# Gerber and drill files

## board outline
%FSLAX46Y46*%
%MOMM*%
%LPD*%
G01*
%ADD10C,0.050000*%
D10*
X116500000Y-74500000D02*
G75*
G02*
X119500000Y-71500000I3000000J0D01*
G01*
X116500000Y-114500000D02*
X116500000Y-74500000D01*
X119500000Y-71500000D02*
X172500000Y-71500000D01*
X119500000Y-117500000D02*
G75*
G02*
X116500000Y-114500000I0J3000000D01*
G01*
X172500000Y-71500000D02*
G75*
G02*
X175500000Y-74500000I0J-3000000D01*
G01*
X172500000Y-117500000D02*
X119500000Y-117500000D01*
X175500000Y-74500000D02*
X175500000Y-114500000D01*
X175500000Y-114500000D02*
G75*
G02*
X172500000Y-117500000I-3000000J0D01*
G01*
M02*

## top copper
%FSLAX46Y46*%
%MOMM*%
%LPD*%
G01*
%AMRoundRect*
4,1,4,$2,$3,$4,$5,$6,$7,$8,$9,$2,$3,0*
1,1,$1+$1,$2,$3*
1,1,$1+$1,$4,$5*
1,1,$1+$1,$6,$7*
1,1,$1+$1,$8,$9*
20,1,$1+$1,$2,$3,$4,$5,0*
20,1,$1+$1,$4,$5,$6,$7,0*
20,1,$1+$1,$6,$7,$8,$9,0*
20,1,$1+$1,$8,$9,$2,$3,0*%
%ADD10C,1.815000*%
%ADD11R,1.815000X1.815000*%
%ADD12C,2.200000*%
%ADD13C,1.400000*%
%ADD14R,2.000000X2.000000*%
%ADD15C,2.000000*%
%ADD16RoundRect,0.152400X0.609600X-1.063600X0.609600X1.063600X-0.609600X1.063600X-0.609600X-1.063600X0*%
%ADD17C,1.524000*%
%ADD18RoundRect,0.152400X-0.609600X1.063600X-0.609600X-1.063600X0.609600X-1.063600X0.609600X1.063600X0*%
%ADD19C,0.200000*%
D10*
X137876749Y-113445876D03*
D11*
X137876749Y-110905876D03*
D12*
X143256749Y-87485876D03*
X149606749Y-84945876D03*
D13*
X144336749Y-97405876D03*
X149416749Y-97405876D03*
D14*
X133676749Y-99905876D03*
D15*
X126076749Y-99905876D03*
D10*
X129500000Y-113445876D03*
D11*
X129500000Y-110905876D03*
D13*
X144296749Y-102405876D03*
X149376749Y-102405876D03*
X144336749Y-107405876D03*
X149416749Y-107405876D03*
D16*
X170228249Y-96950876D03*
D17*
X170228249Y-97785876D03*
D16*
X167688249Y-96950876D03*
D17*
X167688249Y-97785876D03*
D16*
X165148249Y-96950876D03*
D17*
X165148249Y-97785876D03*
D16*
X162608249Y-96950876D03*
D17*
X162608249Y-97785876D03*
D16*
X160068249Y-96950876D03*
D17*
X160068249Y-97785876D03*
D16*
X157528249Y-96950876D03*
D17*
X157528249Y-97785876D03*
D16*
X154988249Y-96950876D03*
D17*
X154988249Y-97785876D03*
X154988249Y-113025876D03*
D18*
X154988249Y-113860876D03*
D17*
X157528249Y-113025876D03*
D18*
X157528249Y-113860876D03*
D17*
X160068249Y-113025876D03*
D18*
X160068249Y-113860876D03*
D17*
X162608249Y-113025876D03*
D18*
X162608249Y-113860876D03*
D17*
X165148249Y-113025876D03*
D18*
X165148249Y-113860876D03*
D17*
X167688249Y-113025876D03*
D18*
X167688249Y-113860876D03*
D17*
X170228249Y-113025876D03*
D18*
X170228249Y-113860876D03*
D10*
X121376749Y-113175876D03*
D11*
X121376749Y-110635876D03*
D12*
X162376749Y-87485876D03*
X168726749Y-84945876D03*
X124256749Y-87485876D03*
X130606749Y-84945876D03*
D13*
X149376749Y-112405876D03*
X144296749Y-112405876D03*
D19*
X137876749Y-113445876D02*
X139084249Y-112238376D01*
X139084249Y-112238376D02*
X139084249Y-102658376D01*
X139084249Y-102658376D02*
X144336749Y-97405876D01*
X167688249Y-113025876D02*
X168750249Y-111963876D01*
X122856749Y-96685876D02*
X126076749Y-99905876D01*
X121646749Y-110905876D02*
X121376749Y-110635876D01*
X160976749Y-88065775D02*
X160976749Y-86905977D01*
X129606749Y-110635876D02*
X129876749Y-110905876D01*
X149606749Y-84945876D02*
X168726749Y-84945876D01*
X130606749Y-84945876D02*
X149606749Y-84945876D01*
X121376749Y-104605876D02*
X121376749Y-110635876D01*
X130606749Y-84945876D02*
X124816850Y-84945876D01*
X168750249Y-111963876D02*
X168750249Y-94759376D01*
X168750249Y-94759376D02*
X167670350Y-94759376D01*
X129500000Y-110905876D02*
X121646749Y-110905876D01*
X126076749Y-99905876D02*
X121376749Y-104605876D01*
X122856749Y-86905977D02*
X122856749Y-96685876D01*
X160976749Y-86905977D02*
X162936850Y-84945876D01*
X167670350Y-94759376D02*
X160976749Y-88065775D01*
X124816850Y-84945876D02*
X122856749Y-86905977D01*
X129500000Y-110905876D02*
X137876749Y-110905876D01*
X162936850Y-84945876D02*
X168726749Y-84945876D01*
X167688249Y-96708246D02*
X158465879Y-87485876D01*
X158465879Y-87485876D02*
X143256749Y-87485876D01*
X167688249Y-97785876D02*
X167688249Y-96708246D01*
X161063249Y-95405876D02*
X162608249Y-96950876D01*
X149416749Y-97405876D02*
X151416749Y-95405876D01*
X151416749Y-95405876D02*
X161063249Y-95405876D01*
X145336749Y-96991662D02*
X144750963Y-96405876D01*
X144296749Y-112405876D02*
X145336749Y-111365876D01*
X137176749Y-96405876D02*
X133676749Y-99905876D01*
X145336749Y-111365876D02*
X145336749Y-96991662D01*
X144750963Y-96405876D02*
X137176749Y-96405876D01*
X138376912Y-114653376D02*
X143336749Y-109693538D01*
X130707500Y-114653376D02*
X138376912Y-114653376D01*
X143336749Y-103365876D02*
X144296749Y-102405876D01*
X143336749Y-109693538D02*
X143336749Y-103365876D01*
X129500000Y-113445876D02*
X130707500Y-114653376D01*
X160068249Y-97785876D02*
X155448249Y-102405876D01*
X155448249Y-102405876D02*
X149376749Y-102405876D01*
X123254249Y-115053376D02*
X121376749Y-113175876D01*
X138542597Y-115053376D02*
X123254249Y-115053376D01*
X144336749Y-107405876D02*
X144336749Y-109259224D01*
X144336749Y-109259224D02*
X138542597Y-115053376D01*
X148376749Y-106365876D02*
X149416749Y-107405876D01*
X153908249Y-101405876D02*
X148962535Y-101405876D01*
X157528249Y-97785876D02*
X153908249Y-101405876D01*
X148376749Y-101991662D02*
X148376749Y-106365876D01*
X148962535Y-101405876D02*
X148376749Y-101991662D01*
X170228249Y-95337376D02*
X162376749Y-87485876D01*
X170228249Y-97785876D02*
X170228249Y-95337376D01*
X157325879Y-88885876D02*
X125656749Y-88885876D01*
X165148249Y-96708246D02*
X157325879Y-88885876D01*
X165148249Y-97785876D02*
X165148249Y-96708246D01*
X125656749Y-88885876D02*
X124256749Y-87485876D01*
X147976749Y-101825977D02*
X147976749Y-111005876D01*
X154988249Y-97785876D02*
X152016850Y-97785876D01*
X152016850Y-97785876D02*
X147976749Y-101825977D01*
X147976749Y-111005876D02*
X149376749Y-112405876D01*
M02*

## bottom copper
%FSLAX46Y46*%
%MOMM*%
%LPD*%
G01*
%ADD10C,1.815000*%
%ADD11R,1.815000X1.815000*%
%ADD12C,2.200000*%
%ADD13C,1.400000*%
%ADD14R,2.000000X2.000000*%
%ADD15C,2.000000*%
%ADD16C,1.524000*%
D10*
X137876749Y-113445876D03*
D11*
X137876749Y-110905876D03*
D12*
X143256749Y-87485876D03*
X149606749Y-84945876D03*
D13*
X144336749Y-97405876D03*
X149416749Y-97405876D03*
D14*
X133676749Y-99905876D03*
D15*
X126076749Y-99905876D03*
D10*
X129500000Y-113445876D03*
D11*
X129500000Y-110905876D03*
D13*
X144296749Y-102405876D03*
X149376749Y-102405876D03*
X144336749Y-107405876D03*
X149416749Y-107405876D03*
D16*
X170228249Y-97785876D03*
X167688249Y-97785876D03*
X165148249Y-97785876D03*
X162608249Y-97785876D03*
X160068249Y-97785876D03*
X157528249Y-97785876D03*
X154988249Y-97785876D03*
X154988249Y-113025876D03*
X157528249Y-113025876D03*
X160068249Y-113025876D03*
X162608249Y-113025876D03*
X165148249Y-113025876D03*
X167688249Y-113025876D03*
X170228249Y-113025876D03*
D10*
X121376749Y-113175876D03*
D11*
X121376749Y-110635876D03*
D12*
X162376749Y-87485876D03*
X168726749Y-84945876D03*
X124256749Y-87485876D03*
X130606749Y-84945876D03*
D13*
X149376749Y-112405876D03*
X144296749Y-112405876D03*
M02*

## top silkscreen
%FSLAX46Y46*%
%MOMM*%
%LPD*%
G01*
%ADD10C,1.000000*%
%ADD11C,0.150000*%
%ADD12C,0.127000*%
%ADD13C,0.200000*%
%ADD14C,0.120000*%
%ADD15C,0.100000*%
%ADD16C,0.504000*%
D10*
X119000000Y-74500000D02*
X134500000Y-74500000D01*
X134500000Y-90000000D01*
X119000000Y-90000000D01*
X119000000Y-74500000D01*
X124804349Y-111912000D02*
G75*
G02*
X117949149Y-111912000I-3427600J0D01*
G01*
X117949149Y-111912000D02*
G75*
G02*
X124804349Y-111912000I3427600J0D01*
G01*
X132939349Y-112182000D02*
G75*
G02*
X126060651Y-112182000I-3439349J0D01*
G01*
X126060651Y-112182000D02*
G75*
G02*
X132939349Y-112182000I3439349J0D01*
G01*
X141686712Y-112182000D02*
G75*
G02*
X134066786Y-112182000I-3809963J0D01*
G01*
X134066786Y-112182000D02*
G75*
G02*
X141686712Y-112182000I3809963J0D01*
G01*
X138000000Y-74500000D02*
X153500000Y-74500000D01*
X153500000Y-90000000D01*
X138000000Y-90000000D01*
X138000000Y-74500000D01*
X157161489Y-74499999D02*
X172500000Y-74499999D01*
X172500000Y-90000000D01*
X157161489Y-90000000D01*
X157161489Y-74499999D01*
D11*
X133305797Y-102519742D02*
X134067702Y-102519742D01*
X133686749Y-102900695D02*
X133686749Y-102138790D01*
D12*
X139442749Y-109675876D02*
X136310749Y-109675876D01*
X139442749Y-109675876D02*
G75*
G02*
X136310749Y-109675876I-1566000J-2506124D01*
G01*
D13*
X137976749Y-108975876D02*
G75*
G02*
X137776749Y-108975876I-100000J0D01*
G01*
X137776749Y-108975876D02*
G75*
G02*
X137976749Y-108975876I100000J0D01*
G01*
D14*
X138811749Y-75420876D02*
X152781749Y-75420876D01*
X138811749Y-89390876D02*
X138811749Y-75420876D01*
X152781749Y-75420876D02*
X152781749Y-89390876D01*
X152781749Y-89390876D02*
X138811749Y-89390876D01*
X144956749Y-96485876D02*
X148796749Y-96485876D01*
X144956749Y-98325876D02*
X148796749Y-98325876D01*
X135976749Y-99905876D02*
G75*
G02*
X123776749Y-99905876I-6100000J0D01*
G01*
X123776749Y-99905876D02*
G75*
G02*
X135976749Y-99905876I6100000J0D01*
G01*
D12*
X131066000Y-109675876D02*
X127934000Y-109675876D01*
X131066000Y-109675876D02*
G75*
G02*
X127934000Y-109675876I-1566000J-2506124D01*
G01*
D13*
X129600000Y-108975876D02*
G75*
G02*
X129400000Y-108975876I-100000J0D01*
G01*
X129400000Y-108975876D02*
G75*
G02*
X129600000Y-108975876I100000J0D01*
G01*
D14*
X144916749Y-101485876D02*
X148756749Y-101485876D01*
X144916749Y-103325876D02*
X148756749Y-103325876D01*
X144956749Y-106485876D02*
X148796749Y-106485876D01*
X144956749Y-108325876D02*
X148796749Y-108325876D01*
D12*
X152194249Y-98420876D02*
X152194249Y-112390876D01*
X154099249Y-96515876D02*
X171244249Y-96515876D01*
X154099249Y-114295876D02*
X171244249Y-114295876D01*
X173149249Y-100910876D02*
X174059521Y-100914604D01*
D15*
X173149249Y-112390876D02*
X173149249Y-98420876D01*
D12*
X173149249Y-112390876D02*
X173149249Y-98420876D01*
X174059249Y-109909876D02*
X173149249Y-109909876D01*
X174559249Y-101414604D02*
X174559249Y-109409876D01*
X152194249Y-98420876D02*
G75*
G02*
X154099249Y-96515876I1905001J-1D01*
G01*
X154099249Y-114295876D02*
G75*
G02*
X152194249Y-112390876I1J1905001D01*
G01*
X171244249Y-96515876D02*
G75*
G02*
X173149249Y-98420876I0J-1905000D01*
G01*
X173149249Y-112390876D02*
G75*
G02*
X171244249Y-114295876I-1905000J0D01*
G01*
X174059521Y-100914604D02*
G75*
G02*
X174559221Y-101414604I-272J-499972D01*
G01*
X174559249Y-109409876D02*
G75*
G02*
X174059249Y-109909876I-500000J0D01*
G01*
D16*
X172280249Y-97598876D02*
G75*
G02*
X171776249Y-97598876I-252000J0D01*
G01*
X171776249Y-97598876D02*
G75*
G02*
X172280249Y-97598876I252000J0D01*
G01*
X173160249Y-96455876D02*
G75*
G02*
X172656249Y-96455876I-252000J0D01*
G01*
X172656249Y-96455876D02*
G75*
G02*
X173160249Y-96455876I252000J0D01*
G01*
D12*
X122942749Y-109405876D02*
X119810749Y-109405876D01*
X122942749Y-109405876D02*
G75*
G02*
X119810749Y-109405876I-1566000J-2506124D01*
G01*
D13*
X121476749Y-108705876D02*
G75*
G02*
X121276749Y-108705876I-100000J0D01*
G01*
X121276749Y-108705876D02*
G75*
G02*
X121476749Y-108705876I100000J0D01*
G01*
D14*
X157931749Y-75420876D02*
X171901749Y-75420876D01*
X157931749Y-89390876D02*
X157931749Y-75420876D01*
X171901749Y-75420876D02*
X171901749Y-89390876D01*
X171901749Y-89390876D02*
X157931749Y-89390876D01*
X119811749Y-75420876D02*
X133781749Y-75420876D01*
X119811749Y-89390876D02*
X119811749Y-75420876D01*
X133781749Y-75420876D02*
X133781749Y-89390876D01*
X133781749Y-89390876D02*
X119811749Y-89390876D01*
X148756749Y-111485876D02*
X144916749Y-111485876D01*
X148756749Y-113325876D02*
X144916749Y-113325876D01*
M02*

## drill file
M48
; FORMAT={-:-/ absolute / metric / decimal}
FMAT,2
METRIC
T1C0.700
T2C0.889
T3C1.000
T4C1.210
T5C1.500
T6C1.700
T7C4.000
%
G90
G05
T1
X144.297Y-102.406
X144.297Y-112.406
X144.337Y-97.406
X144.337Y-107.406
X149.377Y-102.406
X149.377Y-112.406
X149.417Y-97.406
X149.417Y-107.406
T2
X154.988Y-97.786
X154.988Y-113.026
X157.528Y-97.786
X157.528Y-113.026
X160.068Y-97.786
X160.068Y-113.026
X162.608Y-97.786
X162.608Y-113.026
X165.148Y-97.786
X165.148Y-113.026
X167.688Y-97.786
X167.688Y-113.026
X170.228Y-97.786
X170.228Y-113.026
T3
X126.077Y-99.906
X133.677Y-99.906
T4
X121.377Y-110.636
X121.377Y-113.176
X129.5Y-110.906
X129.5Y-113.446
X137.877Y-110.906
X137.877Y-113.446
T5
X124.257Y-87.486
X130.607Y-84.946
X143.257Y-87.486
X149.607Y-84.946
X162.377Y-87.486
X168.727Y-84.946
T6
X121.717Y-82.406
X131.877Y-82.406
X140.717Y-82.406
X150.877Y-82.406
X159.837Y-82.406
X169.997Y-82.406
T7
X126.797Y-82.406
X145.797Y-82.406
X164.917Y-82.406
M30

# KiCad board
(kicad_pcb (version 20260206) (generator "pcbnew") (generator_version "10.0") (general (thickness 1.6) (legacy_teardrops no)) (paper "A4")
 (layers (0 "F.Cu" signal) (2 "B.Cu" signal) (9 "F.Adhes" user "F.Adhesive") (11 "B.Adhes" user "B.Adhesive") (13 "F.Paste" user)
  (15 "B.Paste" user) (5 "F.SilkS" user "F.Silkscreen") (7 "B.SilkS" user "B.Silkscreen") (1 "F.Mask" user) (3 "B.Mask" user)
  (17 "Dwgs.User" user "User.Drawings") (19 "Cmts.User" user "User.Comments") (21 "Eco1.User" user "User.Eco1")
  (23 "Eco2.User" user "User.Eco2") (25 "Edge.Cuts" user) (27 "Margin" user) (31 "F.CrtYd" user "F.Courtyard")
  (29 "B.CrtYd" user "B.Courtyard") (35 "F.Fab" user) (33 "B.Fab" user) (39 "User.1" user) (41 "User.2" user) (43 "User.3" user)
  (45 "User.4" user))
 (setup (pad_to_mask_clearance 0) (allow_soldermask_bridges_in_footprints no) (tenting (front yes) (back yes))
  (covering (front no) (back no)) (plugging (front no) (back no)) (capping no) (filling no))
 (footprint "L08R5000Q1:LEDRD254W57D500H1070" (layer "F.Cu") (at 137.876749 112.175876 -90)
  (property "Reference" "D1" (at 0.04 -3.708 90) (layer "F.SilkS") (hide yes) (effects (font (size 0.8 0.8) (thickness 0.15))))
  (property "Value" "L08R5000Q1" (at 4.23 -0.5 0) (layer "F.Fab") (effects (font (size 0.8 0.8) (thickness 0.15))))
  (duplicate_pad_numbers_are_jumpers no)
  (fp_line (start -2.5 -1.566) (end -2.5 1.566) (stroke (width 0.127) (type solid)) (layer "F.SilkS"))
  (fp_arc (start -2.5 -1.566) (mid 2.961291 0) (end -2.5 1.566) (stroke (width 0.127) (type solid)) (layer "F.SilkS"))
  (fp_circle (center -3.2 0) (end -3.1 0) (stroke (width 0.2) (type solid)) (fill no) (layer "F.SilkS"))
  (pad "A" thru_hole circle (at 1.27 0 270) (size 1.815 1.815) (drill 1.21) (layers "*.Cu" "*.Mask") (remove_unused_layers no)
   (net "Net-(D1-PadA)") (solder_mask_margin 0.102))
  (pad "C" thru_hole rect (at -1.27 0 270) (size 1.815 1.815) (drill 1.21) (layers "*.Cu" "*.Mask") (remove_unused_layers no) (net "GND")
   (solder_mask_margin 0.102)))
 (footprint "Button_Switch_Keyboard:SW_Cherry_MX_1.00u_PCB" (layer "F.Cu") (at 143.256749 87.485876 180)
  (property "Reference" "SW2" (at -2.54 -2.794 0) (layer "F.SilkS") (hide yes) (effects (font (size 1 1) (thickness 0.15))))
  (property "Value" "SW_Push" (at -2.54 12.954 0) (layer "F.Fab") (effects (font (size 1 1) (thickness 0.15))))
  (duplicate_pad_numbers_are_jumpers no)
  (fp_line (start 4.445 12.065) (end -9.525 12.065) (stroke (width 0.12) (type solid)) (layer "F.SilkS"))
  (fp_line (start 4.445 -1.905) (end 4.445 12.065) (stroke (width 0.12) (type solid)) (layer "F.SilkS"))
  (fp_line (start -9.525 12.065) (end -9.525 -1.905) (stroke (width 0.12) (type solid)) (layer "F.SilkS"))
  (fp_line (start -9.525 -1.905) (end 4.445 -1.905) (stroke (width 0.12) (type solid)) (layer "F.SilkS"))
  (pad "" np_thru_hole circle (at -7.62 5.08 180) (size 1.7 1.7) (drill 1.7) (layers "*.Cu" "*.Mask"))
  (pad "" np_thru_hole circle (at -2.54 5.08 180) (size 4 4) (drill 4) (layers "*.Cu" "*.Mask"))
  (pad "" np_thru_hole circle (at 2.54 5.08 180) (size 1.7 1.7) (drill 1.7) (layers "*.Cu" "*.Mask"))
  (pad "1" thru_hole circle (at 0 0 180) (size 2.2 2.2) (drill 1.5) (layers "*.Cu" "*.Mask") (remove_unused_layers no) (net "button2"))
  (pad "2" thru_hole circle (at -6.35 2.54 180) (size 2.2 2.2) (drill 1.5) (layers "*.Cu" "*.Mask") (remove_unused_layers no) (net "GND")))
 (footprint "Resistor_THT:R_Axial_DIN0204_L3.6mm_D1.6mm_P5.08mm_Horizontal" (layer "F.Cu") (at 144.336749 97.405876)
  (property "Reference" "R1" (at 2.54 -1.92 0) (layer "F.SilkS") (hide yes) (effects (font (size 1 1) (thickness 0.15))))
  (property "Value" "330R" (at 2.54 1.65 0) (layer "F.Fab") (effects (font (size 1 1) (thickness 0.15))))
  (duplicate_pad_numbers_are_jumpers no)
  (fp_line (start 0.62 -0.92) (end 4.46 -0.92) (stroke (width 0.12) (type solid)) (layer "F.SilkS"))
  (fp_line (start 0.62 0.92) (end 4.46 0.92) (stroke (width 0.12) (type solid)) (layer "F.SilkS"))
  (pad "1" thru_hole circle (at 0 0) (size 1.4 1.4) (drill 0.7) (layers "*.Cu" "*.Mask") (remove_unused_layers no) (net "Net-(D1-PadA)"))
  (pad "2" thru_hole circle (at 5.08 0) (size 1.4 1.4) (drill 0.7) (layers "*.Cu" "*.Mask") (remove_unused_layers no) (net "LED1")))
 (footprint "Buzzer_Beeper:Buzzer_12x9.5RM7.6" (layer "F.Cu") (at 133.676749 99.905876 180)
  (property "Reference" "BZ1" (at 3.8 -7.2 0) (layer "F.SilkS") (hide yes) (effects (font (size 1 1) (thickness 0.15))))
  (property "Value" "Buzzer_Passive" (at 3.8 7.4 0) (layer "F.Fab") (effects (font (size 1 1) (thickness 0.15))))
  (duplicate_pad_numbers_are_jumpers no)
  (fp_circle (center 3.8 0) (end 9.9 0) (stroke (width 0.12) (type solid)) (fill no) (layer "F.SilkS"))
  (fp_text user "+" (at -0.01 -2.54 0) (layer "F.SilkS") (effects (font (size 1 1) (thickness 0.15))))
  (pad "1" thru_hole rect (at 0 0 180) (size 2 2) (drill 1) (layers "*.Cu" "*.Mask") (remove_unused_layers no) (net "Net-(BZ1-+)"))
  (pad "2" thru_hole circle (at 7.6 0 180) (size 2 2) (drill 1) (layers "*.Cu" "*.Mask") (remove_unused_layers no) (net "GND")))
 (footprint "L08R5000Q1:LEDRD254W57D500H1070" (layer "F.Cu") (at 129.5 112.175876 -90)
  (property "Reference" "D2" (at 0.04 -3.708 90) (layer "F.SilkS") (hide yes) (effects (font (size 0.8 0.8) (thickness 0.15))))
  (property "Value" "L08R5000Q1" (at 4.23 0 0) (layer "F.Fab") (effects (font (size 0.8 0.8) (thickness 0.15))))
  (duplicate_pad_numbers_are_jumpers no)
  (fp_line (start -2.5 -1.566) (end -2.5 1.566) (stroke (width 0.127) (type solid)) (layer "F.SilkS"))
  (fp_arc (start -2.5 -1.566) (mid 2.961291 0) (end -2.5 1.566) (stroke (width 0.127) (type solid)) (layer "F.SilkS"))
  (fp_circle (center -3.2 0) (end -3.1 0) (stroke (width 0.2) (type solid)) (fill no) (layer "F.SilkS"))
  (pad "A" thru_hole circle (at 1.27 0 270) (size 1.815 1.815) (drill 1.21) (layers "*.Cu" "*.Mask") (remove_unused_layers no)
   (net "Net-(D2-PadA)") (solder_mask_margin 0.102))
  (pad "C" thru_hole rect (at -1.27 0 270) (size 1.815 1.815) (drill 1.21) (layers "*.Cu" "*.Mask") (remove_unused_layers no) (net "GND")
   (solder_mask_margin 0.102)))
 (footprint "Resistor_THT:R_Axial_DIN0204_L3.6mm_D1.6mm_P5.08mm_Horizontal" (layer "F.Cu") (at 144.296749 102.405876)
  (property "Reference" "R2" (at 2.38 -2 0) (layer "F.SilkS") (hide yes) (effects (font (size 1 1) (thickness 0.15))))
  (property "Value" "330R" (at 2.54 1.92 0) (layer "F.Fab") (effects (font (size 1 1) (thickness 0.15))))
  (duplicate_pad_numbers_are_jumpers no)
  (fp_line (start 0.62 -0.92) (end 4.46 -0.92) (stroke (width 0.12) (type solid)) (layer "F.SilkS"))
  (fp_line (start 0.62 0.92) (end 4.46 0.92) (stroke (width 0.12) (type solid)) (layer "F.SilkS"))
  (pad "1" thru_hole circle (at 0 0) (size 1.4 1.4) (drill 0.7) (layers "*.Cu" "*.Mask") (remove_unused_layers no) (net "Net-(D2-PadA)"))
  (pad "2" thru_hole circle (at 5.08 0) (size 1.4 1.4) (drill 0.7) (layers "*.Cu" "*.Mask") (remove_unused_layers no) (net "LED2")))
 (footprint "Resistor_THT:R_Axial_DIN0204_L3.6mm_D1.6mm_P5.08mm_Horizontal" (layer "F.Cu") (at 144.336749 107.405876)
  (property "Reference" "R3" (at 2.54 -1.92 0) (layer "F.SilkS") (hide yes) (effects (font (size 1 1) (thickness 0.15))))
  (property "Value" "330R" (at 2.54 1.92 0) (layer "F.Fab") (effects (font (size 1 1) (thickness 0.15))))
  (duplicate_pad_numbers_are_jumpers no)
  (fp_line (start 0.62 -0.92) (end 4.46 -0.92) (stroke (width 0.12) (type solid)) (layer "F.SilkS"))
  (fp_line (start 0.62 0.92) (end 4.46 0.92) (stroke (width 0.12) (type solid)) (layer "F.SilkS"))
  (pad "1" thru_hole circle (at 0 0) (size 1.4 1.4) (drill 0.7) (layers "*.Cu" "*.Mask") (remove_unused_layers no) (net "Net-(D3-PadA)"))
  (pad "2" thru_hole circle (at 5.08 0) (size 1.4 1.4) (drill 0.7) (layers "*.Cu" "*.Mask") (remove_unused_layers no) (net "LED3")))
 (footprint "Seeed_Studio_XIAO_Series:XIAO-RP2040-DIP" (layer "F.Cu") (at 162.608249 105.405876)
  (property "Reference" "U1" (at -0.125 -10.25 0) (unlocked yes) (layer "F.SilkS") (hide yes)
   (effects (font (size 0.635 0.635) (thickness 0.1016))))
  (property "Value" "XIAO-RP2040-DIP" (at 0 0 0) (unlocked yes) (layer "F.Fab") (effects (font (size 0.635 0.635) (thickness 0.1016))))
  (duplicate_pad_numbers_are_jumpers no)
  (fp_line (start -10.414 -6.985) (end -10.414 6.985) (stroke (width 0.127) (type solid)) (layer "F.SilkS"))
  (fp_line (start -8.509 -8.89) (end 8.636 -8.89) (stroke (width 0.127) (type solid)) (layer "F.SilkS"))
  (fp_line (start -8.509 8.89) (end 8.636 8.89) (stroke (width 0.127) (type solid)) (layer "F.SilkS"))
  (fp_line (start 10.541 -4.495) (end 11.451272 -4.491272) (stroke (width 0.127) (type solid)) (layer "F.SilkS"))
  (fp_line (start 10.541 6.985) (end 10.541 -6.985) (stroke (width 0.1) (type solid)) (layer "F.SilkS"))
  (fp_line (start 10.541 6.985) (end 10.541 -6.985) (stroke (width 0.127) (type solid)) (layer "F.SilkS"))
  (fp_line (start 11.451 4.504) (end 10.541 4.504) (stroke (width 0.127) (type solid)) (layer "F.SilkS"))
  (fp_line (start 11.951 -3.991272) (end 11.951 4.004) (stroke (width 0.127) (type solid)) (layer "F.SilkS"))
  (fp_arc (start -10.414 -6.985) (mid -9.856038 -8.332038) (end -8.509 -8.89) (stroke (width 0.127) (type solid)) (layer "F.SilkS"))
  (fp_arc (start -8.509 8.89) (mid -9.856038 8.332038) (end -10.414 6.985) (stroke (width 0.127) (type solid)) (layer "F.SilkS"))
  (fp_arc (start 8.636 -8.89) (mid 9.983038 -8.332038) (end 10.541 -6.985) (stroke (width 0.127) (type solid)) (layer "F.SilkS"))
  (fp_arc (start 10.541 6.985) (mid 9.983038 8.332038) (end 8.636 8.89) (stroke (width 0.127) (type solid)) (layer "F.SilkS"))
  (fp_arc (start 11.451272 -4.491272) (mid 11.804644 -4.344724) (end 11.951 -3.991272) (stroke (width 0.127) (type default))
   (layer "F.SilkS"))
  (fp_arc (start 11.951 4.004) (mid 11.804553 4.357553) (end 11.451 4.504) (stroke (width 0.127) (type default)) (layer "F.SilkS"))
  (fp_circle (center 9.42 -7.807) (end 9.674 -7.807) (stroke (width 0.5) (type solid)) (fill yes) (layer "F.SilkS"))
  (fp_circle (center 10.3 -8.95) (end 10.554 -8.95) (stroke (width 0.5) (type solid)) (fill yes) (layer "F.SilkS"))
  (pad "1" smd roundrect (at 7.62 -8.455 90) (size 2.432 1.524) (layers "F.Cu" "F.Mask") (roundrect_rratio 0.1) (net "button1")
   (thermal_bridge_angle 45))
  (pad "1" thru_hole circle (at 7.62 -7.62 90) (size 1.524 1.524) (drill 0.889) (layers "*.Cu" "*.Mask") (remove_unused_layers no)
   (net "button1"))
  (pad "2" smd roundrect (at 5.08 -8.455 90) (size 2.432 1.524) (layers "F.Cu" "F.Mask") (roundrect_rratio 0.1) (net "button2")
   (thermal_bridge_angle 45))
  (pad "2" thru_hole circle (at 5.08 -7.62 90) (size 1.524 1.524) (drill 0.889) (layers "*.Cu" "*.Mask") (remove_unused_layers no)
   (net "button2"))
  (pad "3" smd roundrect (at 2.54 -8.455 90) (size 2.432 1.524) (layers "F.Cu" "F.Mask") (roundrect_rratio 0.1) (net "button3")
   (thermal_bridge_angle 45))
  (pad "3" thru_hole circle (at 2.54 -7.62 90) (size 1.524 1.524) (drill 0.889) (layers "*.Cu" "*.Mask") (remove_unused_layers no)
   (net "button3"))
  (pad "4" smd roundrect (at 0 -8.455 90) (size 2.432 1.524) (layers "F.Cu" "F.Mask") (roundrect_rratio 0.1) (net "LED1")
   (thermal_bridge_angle 45))
  (pad "4" thru_hole circle (at 0 -7.62 90) (size 1.524 1.524) (drill 0.889) (layers "*.Cu" "*.Mask") (remove_unused_layers no) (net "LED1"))
  (pad "5" smd roundrect (at -2.54 -8.455 90) (size 2.432 1.524) (layers "F.Cu" "F.Mask") (roundrect_rratio 0.1) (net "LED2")
   (thermal_bridge_angle 45))
  (pad "5" thru_hole circle (at -2.54 -7.62 90) (size 1.524 1.524) (drill 0.889) (layers "*.Cu" "*.Mask") (remove_unused_layers no)
   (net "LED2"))
  (pad "6" smd roundrect (at -5.08 -8.455 90) (size 2.432 1.524) (layers "F.Cu" "F.Mask") (roundrect_rratio 0.1) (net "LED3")
   (thermal_bridge_angle 45))
  (pad "6" thru_hole circle (at -5.08 -7.62 90) (size 1.524 1.524) (drill 0.889) (layers "*.Cu" "*.Mask") (remove_unused_layers no)
   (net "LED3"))
  (pad "7" smd roundrect (at -7.62 -8.455 90) (size 2.432 1.524) (layers "F.Cu" "F.Mask") (roundrect_rratio 0.1) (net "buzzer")
   (thermal_bridge_angle 45))
  (pad "7" thru_hole circle (at -7.62 -7.62 90) (size 1.524 1.524) (drill 0.889) (layers "*.Cu" "*.Mask") (remove_unused_layers no)
   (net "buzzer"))
  (pad "8" thru_hole circle (at -7.62 7.62 270) (size 1.524 1.524) (drill 0.889) (layers "*.Cu" "*.Mask") (remove_unused_layers no)
   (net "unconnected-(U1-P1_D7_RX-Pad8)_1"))
  (pad "8" smd roundrect (at -7.62 8.455 270) (size 2.432 1.524) (layers "F.Cu" "F.Mask") (roundrect_rratio 0.1)
   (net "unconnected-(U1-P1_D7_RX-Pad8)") (thermal_bridge_angle 45))
  (pad "9" thru_hole circle (at -5.08 7.62 270) (size 1.524 1.524) (drill 0.889) (layers "*.Cu" "*.Mask") (remove_unused_layers no)
   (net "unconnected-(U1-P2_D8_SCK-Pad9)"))
  (pad "9" smd roundrect (at -5.08 8.455 270) (size 2.432 1.524) (layers "F.Cu" "F.Mask") (roundrect_rratio 0.1)
   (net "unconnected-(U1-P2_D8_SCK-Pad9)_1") (thermal_bridge_angle 45))
  (pad "10" thru_hole circle (at -2.54 7.62 270) (size 1.524 1.524) (drill 0.889) (layers "*.Cu" "*.Mask") (remove_unused_layers no)
   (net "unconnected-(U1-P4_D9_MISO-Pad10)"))
  (pad "10" smd roundrect (at -2.54 8.455 270) (size 2.432 1.524) (layers "F.Cu" "F.Mask") (roundrect_rratio 0.1)
   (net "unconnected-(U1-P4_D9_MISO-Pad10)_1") (thermal_bridge_angle 45))
  (pad "11" thru_hole circle (at 0 7.62 270) (size 1.524 1.524) (drill 0.889) (layers "*.Cu" "*.Mask") (remove_unused_layers no)
   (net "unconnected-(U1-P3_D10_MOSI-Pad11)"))
  (pad "11" smd roundrect (at 0 8.455 270) (size 2.432 1.524) (layers "F.Cu" "F.Mask") (roundrect_rratio 0.1)
   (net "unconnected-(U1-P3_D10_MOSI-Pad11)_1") (thermal_bridge_angle 45))
  (pad "12" thru_hole circle (at 2.54 7.62 270) (size 1.524 1.524) (drill 0.889) (layers "*.Cu" "*.Mask") (remove_unused_layers no)
   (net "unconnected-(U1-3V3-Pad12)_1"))
  (pad "12" smd roundrect (at 2.54 8.455 270) (size 2.432 1.524) (layers "F.Cu" "F.Mask") (roundrect_rratio 0.1)
   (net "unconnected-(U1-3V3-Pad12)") (thermal_bridge_angle 45))
  (pad "13" thru_hole circle (at 5.08 7.62 270) (size 1.524 1.524) (drill 0.889) (layers "*.Cu" "*.Mask") (remove_unused_layers no)
   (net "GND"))
  (pad "13" smd roundrect (at 5.08 8.455 270) (size 2.432 1.524) (layers "F.Cu" "F.Mask") (roundrect_rratio 0.1) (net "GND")
   (thermal_bridge_angle 45))
  (pad "14" thru_hole circle (at 7.62 7.62 270) (size 1.524 1.524) (drill 0.889) (layers "*.Cu" "*.Mask") (remove_unused_layers no)
   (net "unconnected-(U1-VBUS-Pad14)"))
  (pad "14" smd roundrect (at 7.62 8.455 270) (size 2.432 1.524) (layers "F.Cu" "F.Mask") (roundrect_rratio 0.1)
   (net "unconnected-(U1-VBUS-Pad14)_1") (thermal_bridge_angle 45)))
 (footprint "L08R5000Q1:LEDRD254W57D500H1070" (layer "F.Cu") (at 121.376749 111.905876 -90)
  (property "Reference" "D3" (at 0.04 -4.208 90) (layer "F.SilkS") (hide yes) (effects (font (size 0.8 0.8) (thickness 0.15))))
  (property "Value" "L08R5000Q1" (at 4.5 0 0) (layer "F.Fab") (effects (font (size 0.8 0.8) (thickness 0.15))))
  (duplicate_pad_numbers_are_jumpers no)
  (fp_line (start -2.5 -1.566) (end -2.5 1.566) (stroke (width 0.127) (type solid)) (layer "F.SilkS"))
  (fp_arc (start -2.5 -1.566) (mid 2.961291 0) (end -2.5 1.566) (stroke (width 0.127) (type solid)) (layer "F.SilkS"))
  (fp_circle (center -3.2 0) (end -3.1 0) (stroke (width 0.2) (type solid)) (fill no) (layer "F.SilkS"))
  (pad "A" thru_hole circle (at 1.27 0 270) (size 1.815 1.815) (drill 1.21) (layers "*.Cu" "*.Mask") (remove_unused_layers no)
   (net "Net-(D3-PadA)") (solder_mask_margin 0.102))
  (pad "C" thru_hole rect (at -1.27 0 270) (size 1.815 1.815) (drill 1.21) (layers "*.Cu" "*.Mask") (remove_unused_layers no) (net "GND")
   (solder_mask_margin 0.102)))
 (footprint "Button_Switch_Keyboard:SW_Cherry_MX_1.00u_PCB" (layer "F.Cu") (at 162.376749 87.485876 180)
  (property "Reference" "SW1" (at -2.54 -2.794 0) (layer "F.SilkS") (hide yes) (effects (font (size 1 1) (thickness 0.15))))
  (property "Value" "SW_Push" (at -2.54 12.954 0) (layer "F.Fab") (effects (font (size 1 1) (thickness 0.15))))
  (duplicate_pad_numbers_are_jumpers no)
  (fp_line (start 4.445 12.065) (end -9.525 12.065) (stroke (width 0.12) (type solid)) (layer "F.SilkS"))
  (fp_line (start 4.445 -1.905) (end 4.445 12.065) (stroke (width 0.12) (type solid)) (layer "F.SilkS"))
  (fp_line (start -9.525 12.065) (end -9.525 -1.905) (stroke (width 0.12) (type solid)) (layer "F.SilkS"))
  (fp_line (start -9.525 -1.905) (end 4.445 -1.905) (stroke (width 0.12) (type solid)) (layer "F.SilkS"))
  (pad "" np_thru_hole circle (at -7.62 5.08 180) (size 1.7 1.7) (drill 1.7) (layers "*.Cu" "*.Mask"))
  (pad "" np_thru_hole circle (at -2.54 5.08 180) (size 4 4) (drill 4) (layers "*.Cu" "*.Mask"))
  (pad "" np_thru_hole circle (at 2.54 5.08 180) (size 1.7 1.7) (drill 1.7) (layers "*.Cu" "*.Mask"))
  (pad "1" thru_hole circle (at 0 0 180) (size 2.2 2.2) (drill 1.5) (layers "*.Cu" "*.Mask") (remove_unused_layers no) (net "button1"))
  (pad "2" thru_hole circle (at -6.35 2.54 180) (size 2.2 2.2) (drill 1.5) (layers "*.Cu" "*.Mask") (remove_unused_layers no) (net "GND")))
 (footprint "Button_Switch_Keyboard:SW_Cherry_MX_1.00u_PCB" (layer "F.Cu") (at 124.256749 87.485876 180)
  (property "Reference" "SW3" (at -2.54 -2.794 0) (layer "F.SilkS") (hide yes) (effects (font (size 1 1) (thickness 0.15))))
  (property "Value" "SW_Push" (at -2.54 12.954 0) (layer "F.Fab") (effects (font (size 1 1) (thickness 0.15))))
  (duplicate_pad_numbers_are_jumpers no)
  (fp_line (start 4.445 12.065) (end -9.525 12.065) (stroke (width 0.12) (type solid)) (layer "F.SilkS"))
  (fp_line (start 4.445 -1.905) (end 4.445 12.065) (stroke (width 0.12) (type solid)) (layer "F.SilkS"))
  (fp_line (start -9.525 12.065) (end -9.525 -1.905) (stroke (width 0.12) (type solid)) (layer "F.SilkS"))
  (fp_line (start -9.525 -1.905) (end 4.445 -1.905) (stroke (width 0.12) (type solid)) (layer "F.SilkS"))
  (pad "" np_thru_hole circle (at -7.62 5.08 180) (size 1.7 1.7) (drill 1.7) (layers "*.Cu" "*.Mask"))
  (pad "" np_thru_hole circle (at -2.54 5.08 180) (size 4 4) (drill 4) (layers "*.Cu" "*.Mask"))
  (pad "" np_thru_hole circle (at 2.54 5.08 180) (size 1.7 1.7) (drill 1.7) (layers "*.Cu" "*.Mask"))
  (pad "1" thru_hole circle (at 0 0 180) (size 2.2 2.2) (drill 1.5) (layers "*.Cu" "*.Mask") (remove_unused_layers no) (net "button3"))
  (pad "2" thru_hole circle (at -6.35 2.54 180) (size 2.2 2.2) (drill 1.5) (layers "*.Cu" "*.Mask") (remove_unused_layers no) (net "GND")))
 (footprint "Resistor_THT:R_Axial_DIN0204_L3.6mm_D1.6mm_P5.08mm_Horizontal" (layer "F.Cu") (at 149.376749 112.405876 180)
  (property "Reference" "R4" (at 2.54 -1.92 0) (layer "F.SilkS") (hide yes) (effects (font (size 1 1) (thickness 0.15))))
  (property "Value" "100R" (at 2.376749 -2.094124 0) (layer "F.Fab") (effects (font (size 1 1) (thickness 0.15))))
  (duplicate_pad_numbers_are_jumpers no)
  (fp_line (start 0.62 0.92) (end 4.46 0.92) (stroke (width 0.12) (type solid)) (layer "F.SilkS"))
  (fp_line (start 0.62 -0.92) (end 4.46 -0.92) (stroke (width 0.12) (type solid)) (layer "F.SilkS"))
  (pad "1" thru_hole circle (at 0 0 180) (size 1.4 1.4) (drill 0.7) (layers "*.Cu" "*.Mask") (remove_unused_layers no) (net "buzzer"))
  (pad "2" thru_hole circle (at 5.08 0 180) (size 1.4 1.4) (drill 0.7) (layers "*.Cu" "*.Mask") (remove_unused_layers no)
   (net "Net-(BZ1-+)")))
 (gr_rect (start 119 74.5) (end 134.5 90) (stroke (width 1) (type solid)) (fill no) (layer "F.SilkS"))
 (gr_circle (center 121.376749 111.912) (end 124.5 110.5) (stroke (width 1) (type solid)) (fill no) (layer "F.SilkS"))
 (gr_circle (center 129.5 112.182) (end 132.5 110.5) (stroke (width 1) (type solid)) (fill no) (layer "F.SilkS"))
 (gr_circle (center 137.876749 112.182) (end 141 110) (stroke (width 1) (type solid)) (fill no) (layer "F.SilkS"))
 (gr_rect (start 138 74.5) (end 153.5 90) (stroke (width 1) (type solid)) (fill no) (layer "F.SilkS"))
 (gr_rect (start 157.161489 74.499999) (end 172.5 90) (stroke (width 1) (type solid)) (fill no) (layer "F.SilkS"))
 (gr_arc (start 116.5 74.5) (mid 117.37868 72.37868) (end 119.5 71.5) (stroke (width 0.05) (type default)) (layer "Edge.Cuts"))
 (gr_line (start 116.5 114.5) (end 116.5 74.5) (stroke (width 0.05) (type default)) (layer "Edge.Cuts"))
 (gr_line (start 119.5 71.5) (end 172.5 71.5) (stroke (width 0.05) (type default)) (layer "Edge.Cuts"))
 (gr_arc (start 119.5 117.5) (mid 117.37868 116.62132) (end 116.5 114.5) (stroke (width 0.05) (type default)) (layer "Edge.Cuts"))
 (gr_arc (start 172.5 71.5) (mid 174.62132 72.37868) (end 175.5 74.5) (stroke (width 0.05) (type default)) (layer "Edge.Cuts"))
 (gr_line (start 172.5 117.5) (end 119.5 117.5) (stroke (width 0.05) (type default)) (layer "Edge.Cuts"))
 (gr_line (start 175.5 74.5) (end 175.5 114.5) (stroke (width 0.05) (type default)) (layer "Edge.Cuts"))
 (gr_arc (start 175.5 114.5) (mid 174.62132 116.62132) (end 172.5 117.5) (stroke (width 0.05) (type default)) (layer "Edge.Cuts"))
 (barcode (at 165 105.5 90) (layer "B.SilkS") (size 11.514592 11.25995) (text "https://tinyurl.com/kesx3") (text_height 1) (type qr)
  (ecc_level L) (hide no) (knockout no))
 (segment (start 137.876749 113.445876) (end 139.084249 112.238376) (width 0.2) (layer "F.Cu") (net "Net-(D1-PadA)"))
 (segment (start 139.084249 112.238376) (end 139.084249 102.658376) (width 0.2) (layer "F.Cu") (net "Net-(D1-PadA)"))
 (segment (start 139.084249 102.658376) (end 144.336749 97.405876) (width 0.2) (layer "F.Cu") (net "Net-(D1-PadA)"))
 (segment (start 167.688249 113.025876) (end 168.750249 111.963876) (width 0.2) (layer "F.Cu") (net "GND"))
 (segment (start 122.856749 96.685876) (end 126.076749 99.905876) (width 0.2) (layer "F.Cu") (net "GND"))
 (segment (start 121.646749 110.905876) (end 121.376749 110.635876) (width 0.2) (layer "F.Cu") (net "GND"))
 (segment (start 160.976749 88.065775) (end 160.976749 86.905977) (width 0.2) (layer "F.Cu") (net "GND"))
 (segment (start 129.606749 110.635876) (end 129.876749 110.905876) (width 0.2) (layer "F.Cu") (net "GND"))
 (segment (start 149.606749 84.945876) (end 168.726749 84.945876) (width 0.2) (layer "F.Cu") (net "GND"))
 (segment (start 130.606749 84.945876) (end 149.606749 84.945876) (width 0.2) (layer "F.Cu") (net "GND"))
 (segment (start 121.376749 104.605876) (end 121.376749 110.635876) (width 0.2) (layer "F.Cu") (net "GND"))
 (segment (start 130.606749 84.945876) (end 124.81685 84.945876) (width 0.2) (layer "F.Cu") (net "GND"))
 (segment (start 168.750249 111.963876) (end 168.750249 94.759376) (width 0.2) (layer "F.Cu") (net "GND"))
 (segment (start 168.750249 94.759376) (end 167.67035 94.759376) (width 0.2) (layer "F.Cu") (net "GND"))
 (segment (start 129.5 110.905876) (end 121.646749 110.905876) (width 0.2) (layer "F.Cu") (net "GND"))
 (segment (start 126.076749 99.905876) (end 121.376749 104.605876) (width 0.2) (layer "F.Cu") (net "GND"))
 (segment (start 122.856749 86.905977) (end 122.856749 96.685876) (width 0.2) (layer "F.Cu") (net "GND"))
 (segment (start 160.976749 86.905977) (end 162.93685 84.945876) (width 0.2) (layer "F.Cu") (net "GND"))
 (segment (start 167.67035 94.759376) (end 160.976749 88.065775) (width 0.2) (layer "F.Cu") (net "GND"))
 (segment (start 124.81685 84.945876) (end 122.856749 86.905977) (width 0.2) (layer "F.Cu") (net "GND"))
 (segment (start 129.5 110.905876) (end 137.876749 110.905876) (width 0.2) (layer "F.Cu") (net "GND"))
 (segment (start 162.93685 84.945876) (end 168.726749 84.945876) (width 0.2) (layer "F.Cu") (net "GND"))
 (segment (start 167.688249 96.708246) (end 158.465879 87.485876) (width 0.2) (layer "F.Cu") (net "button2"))
 (segment (start 158.465879 87.485876) (end 143.256749 87.485876) (width 0.2) (layer "F.Cu") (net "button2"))
 (segment (start 167.688249 97.785876) (end 167.688249 96.708246) (width 0.2) (layer "F.Cu") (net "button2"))
 (segment (start 161.063249 95.405876) (end 162.608249 96.950876) (width 0.2) (layer "F.Cu") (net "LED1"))
 (segment (start 149.416749 97.405876) (end 151.416749 95.405876) (width 0.2) (layer "F.Cu") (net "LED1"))
 (segment (start 151.416749 95.405876) (end 161.063249 95.405876) (width 0.2) (layer "F.Cu") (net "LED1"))
 (segment (start 145.336749 96.991662) (end 144.750963 96.405876) (width 0.2) (layer "F.Cu") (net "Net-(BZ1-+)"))
 (segment (start 144.296749 112.405876) (end 145.336749 111.365876) (width 0.2) (layer "F.Cu") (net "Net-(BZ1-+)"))
 (segment (start 137.176749 96.405876) (end 133.676749 99.905876) (width 0.2) (layer "F.Cu") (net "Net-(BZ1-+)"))
 (segment (start 145.336749 111.365876) (end 145.336749 96.991662) (width 0.2) (layer "F.Cu") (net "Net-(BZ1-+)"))
 (segment (start 144.750963 96.405876) (end 137.176749 96.405876) (width 0.2) (layer "F.Cu") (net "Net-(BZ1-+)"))
 (segment (start 138.376912 114.653376) (end 143.336749 109.693538) (width 0.2) (layer "F.Cu") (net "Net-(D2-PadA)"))
 (segment (start 130.7075 114.653376) (end 138.376912 114.653376) (width 0.2) (layer "F.Cu") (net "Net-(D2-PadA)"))
 (segment (start 143.336749 103.365876) (end 144.296749 102.405876) (width 0.2) (layer "F.Cu") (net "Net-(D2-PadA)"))
 (segment (start 143.336749 109.693538) (end 143.336749 103.365876) (width 0.2) (layer "F.Cu") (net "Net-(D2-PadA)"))
 (segment (start 129.5 113.445876) (end 130.7075 114.653376) (width 0.2) (layer "F.Cu") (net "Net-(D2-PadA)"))
 (segment (start 160.068249 97.785876) (end 155.448249 102.405876) (width 0.2) (layer "F.Cu") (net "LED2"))
 (segment (start 155.448249 102.405876) (end 149.376749 102.405876) (width 0.2) (layer "F.Cu") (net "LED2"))
 (segment (start 123.254249 115.053376) (end 121.376749 113.175876) (width 0.2) (layer "F.Cu") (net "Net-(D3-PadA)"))
 (segment (start 138.542597 115.053376) (end 123.254249 115.053376) (width 0.2) (layer "F.Cu") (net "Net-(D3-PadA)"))
 (segment (start 144.336749 107.405876) (end 144.336749 109.259224) (width 0.2) (layer "F.Cu") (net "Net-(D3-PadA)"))
 (segment (start 144.336749 109.259224) (end 138.542597 115.053376) (width 0.2) (layer "F.Cu") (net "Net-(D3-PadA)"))
 (segment (start 148.376749 106.365876) (end 149.416749 107.405876) (width 0.2) (layer "F.Cu") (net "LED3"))
 (segment (start 153.908249 101.405876) (end 148.962535 101.405876) (width 0.2) (layer "F.Cu") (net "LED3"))
 (segment (start 157.528249 97.785876) (end 153.908249 101.405876) (width 0.2) (layer "F.Cu") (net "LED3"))
 (segment (start 148.376749 101.991662) (end 148.376749 106.365876) (width 0.2) (layer "F.Cu") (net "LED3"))
 (segment (start 148.962535 101.405876) (end 148.376749 101.991662) (width 0.2) (layer "F.Cu") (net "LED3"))
 (segment (start 170.228249 95.337376) (end 162.376749 87.485876) (width 0.2) (layer "F.Cu") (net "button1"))
 (segment (start 170.228249 97.785876) (end 170.228249 95.337376) (width 0.2) (layer "F.Cu") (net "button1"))
 (segment (start 157.325879 88.885876) (end 125.656749 88.885876) (width 0.2) (layer "F.Cu") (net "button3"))
 (segment (start 165.148249 96.708246) (end 157.325879 88.885876) (width 0.2) (layer "F.Cu") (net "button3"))
 (segment (start 165.148249 97.785876) (end 165.148249 96.708246) (width 0.2) (layer "F.Cu") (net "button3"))
 (segment (start 125.656749 88.885876) (end 124.256749 87.485876) (width 0.2) (layer "F.Cu") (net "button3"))
 (segment (start 147.976749 101.825977) (end 147.976749 111.005876) (width 0.2) (layer "F.Cu") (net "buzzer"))
 (segment (start 154.988249 97.785876) (end 152.01685 97.785876) (width 0.2) (layer "F.Cu") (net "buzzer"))
 (segment (start 152.01685 97.785876) (end 147.976749 101.825977) (width 0.2) (layer "F.Cu") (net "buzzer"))
 (segment (start 147.976749 111.005876) (end 149.376749 112.405876) (width 0.2) (layer "F.Cu") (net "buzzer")))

